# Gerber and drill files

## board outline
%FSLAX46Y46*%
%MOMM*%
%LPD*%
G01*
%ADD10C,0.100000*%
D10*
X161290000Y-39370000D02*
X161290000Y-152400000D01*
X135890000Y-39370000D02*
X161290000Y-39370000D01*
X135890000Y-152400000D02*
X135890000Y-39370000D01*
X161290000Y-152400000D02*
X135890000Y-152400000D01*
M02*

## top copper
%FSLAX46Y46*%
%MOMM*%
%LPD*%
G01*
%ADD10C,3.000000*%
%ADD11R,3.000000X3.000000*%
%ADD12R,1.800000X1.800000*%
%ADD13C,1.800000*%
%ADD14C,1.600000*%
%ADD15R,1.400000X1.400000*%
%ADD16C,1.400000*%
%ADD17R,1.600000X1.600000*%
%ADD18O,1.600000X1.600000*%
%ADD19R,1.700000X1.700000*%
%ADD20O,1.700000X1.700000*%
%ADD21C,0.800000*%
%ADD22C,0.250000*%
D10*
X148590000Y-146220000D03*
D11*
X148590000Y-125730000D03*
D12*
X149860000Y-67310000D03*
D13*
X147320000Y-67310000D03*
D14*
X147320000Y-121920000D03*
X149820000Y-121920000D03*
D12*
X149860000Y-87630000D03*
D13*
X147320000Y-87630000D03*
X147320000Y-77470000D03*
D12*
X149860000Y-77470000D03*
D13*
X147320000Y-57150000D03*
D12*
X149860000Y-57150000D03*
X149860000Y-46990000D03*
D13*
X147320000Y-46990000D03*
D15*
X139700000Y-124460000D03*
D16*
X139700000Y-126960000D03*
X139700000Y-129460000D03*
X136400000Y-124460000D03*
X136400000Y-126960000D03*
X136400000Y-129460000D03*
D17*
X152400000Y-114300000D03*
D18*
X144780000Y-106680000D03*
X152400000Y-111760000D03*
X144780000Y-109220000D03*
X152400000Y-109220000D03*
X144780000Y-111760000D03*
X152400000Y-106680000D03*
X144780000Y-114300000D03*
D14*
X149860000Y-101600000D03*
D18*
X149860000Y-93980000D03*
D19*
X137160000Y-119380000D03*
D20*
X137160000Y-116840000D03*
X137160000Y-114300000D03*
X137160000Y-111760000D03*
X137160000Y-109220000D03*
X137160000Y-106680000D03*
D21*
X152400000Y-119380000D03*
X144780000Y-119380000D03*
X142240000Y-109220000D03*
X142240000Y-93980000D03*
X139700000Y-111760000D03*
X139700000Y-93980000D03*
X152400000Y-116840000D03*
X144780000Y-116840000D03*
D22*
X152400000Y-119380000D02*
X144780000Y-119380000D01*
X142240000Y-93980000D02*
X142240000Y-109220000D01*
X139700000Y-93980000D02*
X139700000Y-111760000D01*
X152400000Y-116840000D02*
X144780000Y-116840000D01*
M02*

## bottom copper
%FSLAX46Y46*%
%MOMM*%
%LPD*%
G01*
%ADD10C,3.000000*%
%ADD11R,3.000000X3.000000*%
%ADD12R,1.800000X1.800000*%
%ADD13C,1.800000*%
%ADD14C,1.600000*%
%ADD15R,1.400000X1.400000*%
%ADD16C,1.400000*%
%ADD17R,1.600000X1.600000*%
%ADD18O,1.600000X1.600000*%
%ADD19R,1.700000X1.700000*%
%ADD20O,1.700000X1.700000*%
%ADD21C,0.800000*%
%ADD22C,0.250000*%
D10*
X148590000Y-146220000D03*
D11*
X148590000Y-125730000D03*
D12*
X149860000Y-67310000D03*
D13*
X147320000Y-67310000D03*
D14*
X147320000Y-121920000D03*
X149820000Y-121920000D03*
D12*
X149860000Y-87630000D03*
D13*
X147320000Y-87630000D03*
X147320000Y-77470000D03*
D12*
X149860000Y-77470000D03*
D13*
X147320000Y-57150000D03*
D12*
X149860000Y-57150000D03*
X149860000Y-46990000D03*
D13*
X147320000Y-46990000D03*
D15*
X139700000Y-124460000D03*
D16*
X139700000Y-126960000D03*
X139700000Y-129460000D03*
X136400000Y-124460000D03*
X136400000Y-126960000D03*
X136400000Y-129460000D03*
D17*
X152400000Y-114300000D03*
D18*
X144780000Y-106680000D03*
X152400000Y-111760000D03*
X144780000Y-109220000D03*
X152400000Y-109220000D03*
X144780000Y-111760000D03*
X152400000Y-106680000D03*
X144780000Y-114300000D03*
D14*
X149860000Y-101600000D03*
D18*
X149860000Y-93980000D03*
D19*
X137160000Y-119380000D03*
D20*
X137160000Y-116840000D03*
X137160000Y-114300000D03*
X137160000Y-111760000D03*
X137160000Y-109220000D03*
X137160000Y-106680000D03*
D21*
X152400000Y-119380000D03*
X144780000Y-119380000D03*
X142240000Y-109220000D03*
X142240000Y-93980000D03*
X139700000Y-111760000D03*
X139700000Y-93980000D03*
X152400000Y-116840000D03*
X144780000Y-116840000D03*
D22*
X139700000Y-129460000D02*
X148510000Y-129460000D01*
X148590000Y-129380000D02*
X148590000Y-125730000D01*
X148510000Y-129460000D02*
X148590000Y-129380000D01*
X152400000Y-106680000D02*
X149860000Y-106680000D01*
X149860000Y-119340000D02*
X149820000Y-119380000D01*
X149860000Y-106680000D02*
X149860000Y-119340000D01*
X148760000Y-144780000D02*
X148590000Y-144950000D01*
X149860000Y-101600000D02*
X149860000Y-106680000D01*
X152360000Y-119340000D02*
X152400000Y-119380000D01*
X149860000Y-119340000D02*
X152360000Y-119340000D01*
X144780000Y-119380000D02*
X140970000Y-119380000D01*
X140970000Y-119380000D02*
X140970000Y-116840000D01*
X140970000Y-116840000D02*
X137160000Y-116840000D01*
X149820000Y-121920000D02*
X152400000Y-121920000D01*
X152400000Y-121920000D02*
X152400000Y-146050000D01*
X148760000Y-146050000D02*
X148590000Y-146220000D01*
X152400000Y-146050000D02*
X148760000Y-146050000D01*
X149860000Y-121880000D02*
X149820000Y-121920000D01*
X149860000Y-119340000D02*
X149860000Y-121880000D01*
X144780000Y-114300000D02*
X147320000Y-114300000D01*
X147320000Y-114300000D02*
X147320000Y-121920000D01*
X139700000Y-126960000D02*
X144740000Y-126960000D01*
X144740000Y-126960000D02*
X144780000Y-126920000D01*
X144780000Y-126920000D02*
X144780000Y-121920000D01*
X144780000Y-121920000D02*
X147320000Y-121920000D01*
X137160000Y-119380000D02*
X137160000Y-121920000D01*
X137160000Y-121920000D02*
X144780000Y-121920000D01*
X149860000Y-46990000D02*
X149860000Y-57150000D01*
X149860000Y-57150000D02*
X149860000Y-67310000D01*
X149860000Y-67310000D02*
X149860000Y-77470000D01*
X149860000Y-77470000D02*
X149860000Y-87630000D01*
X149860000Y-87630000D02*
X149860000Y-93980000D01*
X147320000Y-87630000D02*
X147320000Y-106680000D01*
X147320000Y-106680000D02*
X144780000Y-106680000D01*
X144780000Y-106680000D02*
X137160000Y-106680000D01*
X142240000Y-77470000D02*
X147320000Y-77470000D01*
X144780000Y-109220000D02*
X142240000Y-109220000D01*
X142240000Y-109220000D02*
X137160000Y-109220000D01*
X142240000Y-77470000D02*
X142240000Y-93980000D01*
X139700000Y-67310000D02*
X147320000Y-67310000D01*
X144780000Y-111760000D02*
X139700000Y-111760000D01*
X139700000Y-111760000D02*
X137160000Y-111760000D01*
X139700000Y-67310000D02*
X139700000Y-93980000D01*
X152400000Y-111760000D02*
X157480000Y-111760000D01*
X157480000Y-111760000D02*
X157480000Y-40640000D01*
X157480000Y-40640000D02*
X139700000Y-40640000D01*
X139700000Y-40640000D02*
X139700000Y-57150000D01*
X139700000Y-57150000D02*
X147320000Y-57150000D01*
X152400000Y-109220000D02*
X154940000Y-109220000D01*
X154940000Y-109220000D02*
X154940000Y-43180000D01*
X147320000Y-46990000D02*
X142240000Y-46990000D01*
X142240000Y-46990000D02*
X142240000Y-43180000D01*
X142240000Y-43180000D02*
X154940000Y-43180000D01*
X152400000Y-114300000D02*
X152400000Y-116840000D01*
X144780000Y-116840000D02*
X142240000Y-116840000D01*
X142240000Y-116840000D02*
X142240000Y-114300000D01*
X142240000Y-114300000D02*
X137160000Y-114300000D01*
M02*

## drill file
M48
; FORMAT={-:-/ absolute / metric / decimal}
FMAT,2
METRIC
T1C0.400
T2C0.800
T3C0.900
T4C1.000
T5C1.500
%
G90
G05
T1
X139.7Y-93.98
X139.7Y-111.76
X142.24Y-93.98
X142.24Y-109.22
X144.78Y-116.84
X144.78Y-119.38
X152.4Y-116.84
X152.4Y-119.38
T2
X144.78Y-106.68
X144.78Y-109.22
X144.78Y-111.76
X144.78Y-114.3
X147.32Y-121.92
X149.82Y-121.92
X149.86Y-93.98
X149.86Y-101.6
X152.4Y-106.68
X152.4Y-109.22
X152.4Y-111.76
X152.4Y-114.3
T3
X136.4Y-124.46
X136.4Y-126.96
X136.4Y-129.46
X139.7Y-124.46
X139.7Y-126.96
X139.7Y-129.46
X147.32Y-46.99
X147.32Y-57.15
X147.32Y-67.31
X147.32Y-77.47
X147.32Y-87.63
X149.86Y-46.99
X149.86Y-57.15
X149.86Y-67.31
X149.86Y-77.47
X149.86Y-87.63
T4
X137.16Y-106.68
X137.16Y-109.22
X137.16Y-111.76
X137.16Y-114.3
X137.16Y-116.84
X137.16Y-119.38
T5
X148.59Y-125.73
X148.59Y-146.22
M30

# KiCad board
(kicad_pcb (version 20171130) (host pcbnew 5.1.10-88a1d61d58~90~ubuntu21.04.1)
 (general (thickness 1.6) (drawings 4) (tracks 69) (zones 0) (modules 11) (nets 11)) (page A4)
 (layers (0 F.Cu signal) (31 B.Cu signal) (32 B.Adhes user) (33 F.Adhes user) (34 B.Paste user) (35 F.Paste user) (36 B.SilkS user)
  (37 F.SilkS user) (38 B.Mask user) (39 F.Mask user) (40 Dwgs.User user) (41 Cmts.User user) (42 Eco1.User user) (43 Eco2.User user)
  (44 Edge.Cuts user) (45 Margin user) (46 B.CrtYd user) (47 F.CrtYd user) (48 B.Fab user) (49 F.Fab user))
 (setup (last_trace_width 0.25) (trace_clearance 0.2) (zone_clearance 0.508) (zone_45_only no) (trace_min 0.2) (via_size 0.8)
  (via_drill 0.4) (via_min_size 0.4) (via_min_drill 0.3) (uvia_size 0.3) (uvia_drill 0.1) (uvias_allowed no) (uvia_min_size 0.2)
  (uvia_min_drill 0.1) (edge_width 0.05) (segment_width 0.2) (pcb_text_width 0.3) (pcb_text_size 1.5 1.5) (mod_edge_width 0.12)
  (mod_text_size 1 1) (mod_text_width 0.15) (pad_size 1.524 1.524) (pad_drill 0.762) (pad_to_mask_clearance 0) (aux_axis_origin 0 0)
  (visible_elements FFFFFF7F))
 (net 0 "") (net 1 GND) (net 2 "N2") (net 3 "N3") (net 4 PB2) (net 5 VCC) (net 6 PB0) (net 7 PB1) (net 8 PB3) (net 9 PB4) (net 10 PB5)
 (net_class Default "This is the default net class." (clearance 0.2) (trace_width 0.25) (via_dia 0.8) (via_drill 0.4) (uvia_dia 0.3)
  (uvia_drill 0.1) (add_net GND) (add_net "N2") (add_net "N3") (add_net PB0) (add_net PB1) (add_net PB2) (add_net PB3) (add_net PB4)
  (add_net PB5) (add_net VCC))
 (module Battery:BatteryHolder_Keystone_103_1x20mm (layer F.Cu) (at 148.59 125.73 270)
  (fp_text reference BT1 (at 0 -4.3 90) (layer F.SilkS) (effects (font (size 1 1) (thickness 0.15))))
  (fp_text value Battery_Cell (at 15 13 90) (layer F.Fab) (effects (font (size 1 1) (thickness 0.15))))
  (pad 2 thru_hole circle (at 20.49 0 270) (size 3 3) (drill 1.5) (layers *.Cu *.Mask) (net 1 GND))
  (pad 1 thru_hole rect (at 0 0 270) (size 3 3) (drill 1.5) (layers *.Cu *.Mask) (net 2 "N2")))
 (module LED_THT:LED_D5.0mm (layer F.Cu) (at 149.86 67.31 180)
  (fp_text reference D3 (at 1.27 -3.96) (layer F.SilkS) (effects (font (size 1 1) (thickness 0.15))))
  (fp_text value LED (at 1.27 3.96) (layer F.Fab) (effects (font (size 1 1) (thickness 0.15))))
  (pad 1 thru_hole rect (at 0 0 180) (size 1.8 1.8) (drill 0.9) (layers *.Cu *.Mask) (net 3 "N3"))
  (pad 2 thru_hole circle (at 2.54 0 180) (size 1.8 1.8) (drill 0.9) (layers *.Cu *.Mask) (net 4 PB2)))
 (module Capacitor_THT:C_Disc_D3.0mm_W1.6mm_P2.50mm (layer F.Cu) (at 147.32 121.92)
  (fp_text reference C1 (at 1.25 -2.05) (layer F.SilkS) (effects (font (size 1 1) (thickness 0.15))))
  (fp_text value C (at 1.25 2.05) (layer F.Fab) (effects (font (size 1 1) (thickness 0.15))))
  (pad 1 thru_hole circle (at 0 0) (size 1.6 1.6) (drill 0.8) (layers *.Cu *.Mask) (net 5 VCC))
  (pad 2 thru_hole circle (at 2.5 0) (size 1.6 1.6) (drill 0.8) (layers *.Cu *.Mask) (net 1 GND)))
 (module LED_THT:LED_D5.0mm (layer F.Cu) (at 149.86 87.63 180)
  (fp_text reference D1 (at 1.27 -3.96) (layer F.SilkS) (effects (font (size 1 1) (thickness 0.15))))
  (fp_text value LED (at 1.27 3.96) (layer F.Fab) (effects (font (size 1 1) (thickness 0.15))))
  (pad 1 thru_hole rect (at 0 0 180) (size 1.8 1.8) (drill 0.9) (layers *.Cu *.Mask) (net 3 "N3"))
  (pad 2 thru_hole circle (at 2.54 0 180) (size 1.8 1.8) (drill 0.9) (layers *.Cu *.Mask) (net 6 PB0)))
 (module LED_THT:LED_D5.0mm (layer F.Cu) (at 149.86 77.47 180)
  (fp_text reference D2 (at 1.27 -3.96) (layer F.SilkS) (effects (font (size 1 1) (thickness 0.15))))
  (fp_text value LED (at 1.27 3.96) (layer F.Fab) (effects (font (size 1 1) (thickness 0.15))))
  (pad 2 thru_hole circle (at 2.54 0 180) (size 1.8 1.8) (drill 0.9) (layers *.Cu *.Mask) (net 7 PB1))
  (pad 1 thru_hole rect (at 0 0 180) (size 1.8 1.8) (drill 0.9) (layers *.Cu *.Mask) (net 3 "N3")))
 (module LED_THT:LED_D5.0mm (layer F.Cu) (at 149.86 57.15 180)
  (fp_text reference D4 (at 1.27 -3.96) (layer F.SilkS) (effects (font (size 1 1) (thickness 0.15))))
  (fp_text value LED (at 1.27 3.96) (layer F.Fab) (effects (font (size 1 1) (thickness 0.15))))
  (pad 2 thru_hole circle (at 2.54 0 180) (size 1.8 1.8) (drill 0.9) (layers *.Cu *.Mask) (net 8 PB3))
  (pad 1 thru_hole rect (at 0 0 180) (size 1.8 1.8) (drill 0.9) (layers *.Cu *.Mask) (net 3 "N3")))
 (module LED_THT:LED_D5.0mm (layer F.Cu) (at 149.86 46.99 180)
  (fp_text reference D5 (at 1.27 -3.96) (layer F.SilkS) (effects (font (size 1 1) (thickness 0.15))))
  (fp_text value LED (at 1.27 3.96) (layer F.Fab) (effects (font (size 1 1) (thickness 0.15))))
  (pad 1 thru_hole rect (at 0 0 180) (size 1.8 1.8) (drill 0.9) (layers *.Cu *.Mask) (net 3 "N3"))
  (pad 2 thru_hole circle (at 2.54 0 180) (size 1.8 1.8) (drill 0.9) (layers *.Cu *.Mask) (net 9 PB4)))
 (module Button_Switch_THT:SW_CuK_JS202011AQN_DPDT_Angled (layer F.Cu) (at 139.7 124.46 270)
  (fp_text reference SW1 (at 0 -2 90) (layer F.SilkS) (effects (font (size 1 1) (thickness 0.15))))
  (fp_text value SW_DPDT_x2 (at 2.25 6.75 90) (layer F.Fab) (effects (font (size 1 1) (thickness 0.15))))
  (pad 1 thru_hole rect (at 0 0 270) (size 1.4 1.4) (drill 0.9) (layers *.Cu *.Mask))
  (pad 2 thru_hole circle (at 2.5 0 270) (size 1.4 1.4) (drill 0.9) (layers *.Cu *.Mask) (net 5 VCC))
  (pad 3 thru_hole circle (at 5 0 270) (size 1.4 1.4) (drill 0.9) (layers *.Cu *.Mask) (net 2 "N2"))
  (pad 4 thru_hole circle (at 0 3.3 270) (size 1.4 1.4) (drill 0.9) (layers *.Cu *.Mask))
  (pad 5 thru_hole circle (at 2.5 3.3 270) (size 1.4 1.4) (drill 0.9) (layers *.Cu *.Mask))
  (pad 6 thru_hole circle (at 5 3.3 270) (size 1.4 1.4) (drill 0.9) (layers *.Cu *.Mask)))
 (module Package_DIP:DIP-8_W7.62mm (layer F.Cu) (at 152.4 114.3 180)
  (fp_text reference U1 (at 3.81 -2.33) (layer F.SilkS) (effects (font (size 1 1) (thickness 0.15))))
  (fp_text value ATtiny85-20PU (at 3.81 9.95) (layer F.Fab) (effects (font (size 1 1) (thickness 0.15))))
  (pad 1 thru_hole rect (at 0 0 180) (size 1.6 1.6) (drill 0.8) (layers *.Cu *.Mask) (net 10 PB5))
  (pad 5 thru_hole oval (at 7.62 7.62 180) (size 1.6 1.6) (drill 0.8) (layers *.Cu *.Mask) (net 6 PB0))
  (pad 2 thru_hole oval (at 0 2.54 180) (size 1.6 1.6) (drill 0.8) (layers *.Cu *.Mask) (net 8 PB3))
  (pad 6 thru_hole oval (at 7.62 5.08 180) (size 1.6 1.6) (drill 0.8) (layers *.Cu *.Mask) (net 7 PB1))
  (pad 3 thru_hole oval (at 0 5.08 180) (size 1.6 1.6) (drill 0.8) (layers *.Cu *.Mask) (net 9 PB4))
  (pad 7 thru_hole oval (at 7.62 2.54 180) (size 1.6 1.6) (drill 0.8) (layers *.Cu *.Mask) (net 4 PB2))
  (pad 4 thru_hole oval (at 0 7.62 180) (size 1.6 1.6) (drill 0.8) (layers *.Cu *.Mask) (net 1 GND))
  (pad 8 thru_hole oval (at 7.62 0 180) (size 1.6 1.6) (drill 0.8) (layers *.Cu *.Mask) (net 5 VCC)))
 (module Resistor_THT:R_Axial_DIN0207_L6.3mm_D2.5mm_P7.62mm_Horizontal (layer F.Cu) (at 149.86 101.6 90)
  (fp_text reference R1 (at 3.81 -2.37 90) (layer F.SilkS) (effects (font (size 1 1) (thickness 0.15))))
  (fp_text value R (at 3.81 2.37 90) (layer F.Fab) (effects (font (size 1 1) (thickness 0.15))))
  (pad 1 thru_hole circle (at 0 0 90) (size 1.6 1.6) (drill 0.8) (layers *.Cu *.Mask) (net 1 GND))
  (pad 2 thru_hole oval (at 7.62 0 90) (size 1.6 1.6) (drill 0.8) (layers *.Cu *.Mask) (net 3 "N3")))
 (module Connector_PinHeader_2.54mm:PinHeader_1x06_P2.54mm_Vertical (layer F.Cu) (at 137.16 119.38 180)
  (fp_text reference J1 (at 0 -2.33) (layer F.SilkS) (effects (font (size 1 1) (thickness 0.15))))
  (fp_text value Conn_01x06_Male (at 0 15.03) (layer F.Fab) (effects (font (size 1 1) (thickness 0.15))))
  (pad 1 thru_hole rect (at 0 0 180) (size 1.7 1.7) (drill 1) (layers *.Cu *.Mask) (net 5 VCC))
  (pad 2 thru_hole oval (at 0 2.54 180) (size 1.7 1.7) (drill 1) (layers *.Cu *.Mask) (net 1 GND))
  (pad 3 thru_hole oval (at 0 5.08 180) (size 1.7 1.7) (drill 1) (layers *.Cu *.Mask) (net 10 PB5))
  (pad 4 thru_hole oval (at 0 7.62 180) (size 1.7 1.7) (drill 1) (layers *.Cu *.Mask) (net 4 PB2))
  (pad 5 thru_hole oval (at 0 10.16 180) (size 1.7 1.7) (drill 1) (layers *.Cu *.Mask) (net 7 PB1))
  (pad 6 thru_hole oval (at 0 12.7 180) (size 1.7 1.7) (drill 1) (layers *.Cu *.Mask) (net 6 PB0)))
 (gr_line (start 161.29 39.37) (end 161.29 152.4) (layer Edge.Cuts) (width 0.1))
 (gr_line (start 135.89 39.37) (end 161.29 39.37) (layer Edge.Cuts) (width 0.1))
 (gr_line (start 135.89 152.4) (end 135.89 39.37) (layer Edge.Cuts) (width 0.1))
 (gr_line (start 161.29 152.4) (end 135.89 152.4) (layer Edge.Cuts) (width 0.1))
 (segment (start 139.7 129.46) (end 148.51 129.46) (width 0.25) (layer B.Cu) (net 2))
 (segment (start 148.59 129.38) (end 148.59 125.73) (width 0.25) (layer B.Cu) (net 2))
 (segment (start 148.51 129.46) (end 148.59 129.38) (width 0.25) (layer B.Cu) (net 2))
 (segment (start 152.4 106.68) (end 149.86 106.68) (width 0.25) (layer B.Cu) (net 1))
 (segment (start 149.86 119.34) (end 149.82 119.38) (width 0.25) (layer B.Cu) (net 1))
 (segment (start 149.86 106.68) (end 149.86 119.34) (width 0.25) (layer B.Cu) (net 1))
 (segment (start 148.76 144.78) (end 148.59 144.95) (width 0.25) (layer B.Cu) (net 1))
 (segment (start 149.86 101.6) (end 149.86 106.68) (width 0.25) (layer B.Cu) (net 1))
 (via (at 152.4 119.38) (size 0.8) (drill 0.4) (layers F.Cu B.Cu) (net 1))
 (segment (start 152.36 119.34) (end 152.4 119.38) (width 0.25) (layer B.Cu) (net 1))
 (segment (start 149.86 119.34) (end 152.36 119.34) (width 0.25) (layer B.Cu) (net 1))
 (via (at 144.78 119.38) (size 0.8) (drill 0.4) (layers F.Cu B.Cu) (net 1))
 (segment (start 152.4 119.38) (end 144.78 119.38) (width 0.25) (layer F.Cu) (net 1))
 (segment (start 144.78 119.38) (end 140.97 119.38) (width 0.25) (layer B.Cu) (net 1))
 (segment (start 140.97 119.38) (end 140.97 116.84) (width 0.25) (layer B.Cu) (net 1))
 (segment (start 140.97 116.84) (end 137.16 116.84) (width 0.25) (layer B.Cu) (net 1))
 (segment (start 149.82 121.92) (end 152.4 121.92) (width 0.25) (layer B.Cu) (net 1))
 (segment (start 152.4 121.92) (end 152.4 146.05) (width 0.25) (layer B.Cu) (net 1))
 (segment (start 148.76 146.05) (end 148.59 146.22) (width 0.25) (layer B.Cu) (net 1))
 (segment (start 152.4 146.05) (end 148.76 146.05) (width 0.25) (layer B.Cu) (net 1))
 (segment (start 149.86 121.88) (end 149.82 121.92) (width 0.25) (layer B.Cu) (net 1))
 (segment (start 149.86 119.34) (end 149.86 121.88) (width 0.25) (layer B.Cu) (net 1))
 (segment (start 144.78 114.3) (end 147.32 114.3) (width 0.25) (layer B.Cu) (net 5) (status 10))
 (segment (start 147.32 114.3) (end 147.32 121.92) (width 0.25) (layer B.Cu) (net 5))
 (segment (start 139.7 126.96) (end 144.74 126.96) (width 0.25) (layer B.Cu) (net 5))
 (segment (start 144.74 126.96) (end 144.78 126.92) (width 0.25) (layer B.Cu) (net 5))
 (segment (start 144.78 126.92) (end 144.78 121.92) (width 0.25) (layer B.Cu) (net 5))
 (segment (start 144.78 121.92) (end 147.32 121.92) (width 0.25) (layer B.Cu) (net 5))
 (segment (start 137.16 119.38) (end 137.16 121.92) (width 0.25) (layer B.Cu) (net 5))
 (segment (start 137.16 121.92) (end 144.78 121.92) (width 0.25) (layer B.Cu) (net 5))
 (segment (start 149.86 46.99) (end 149.86 57.15) (width 0.25) (layer B.Cu) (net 3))
 (segment (start 149.86 57.15) (end 149.86 67.31) (width 0.25) (layer B.Cu) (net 3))
 (segment (start 149.86 67.31) (end 149.86 77.47) (width 0.25) (layer B.Cu) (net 3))
 (segment (start 149.86 77.47) (end 149.86 87.63) (width 0.25) (layer B.Cu) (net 3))
 (segment (start 149.86 87.63) (end 149.86 93.98) (width 0.25) (layer B.Cu) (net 3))
 (segment (start 147.32 87.63) (end 147.32 106.68) (width 0.25) (layer B.Cu) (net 6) (status 10))
 (segment (start 147.32 106.68) (end 144.78 106.68) (width 0.25) (layer B.Cu) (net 6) (status 20))
 (segment (start 144.78 106.68) (end 137.16 106.68) (width 0.25) (layer B.Cu) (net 6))
 (segment (start 142.24 77.47) (end 147.32 77.47) (width 0.25) (layer B.Cu) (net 7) (status 20))
 (segment (start 144.78 109.22) (end 142.24 109.22) (width 0.25) (layer B.Cu) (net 7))
 (segment (start 142.24 109.22) (end 137.16 109.22) (width 0.25) (layer B.Cu) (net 7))
 (via (at 142.24 109.22) (size 0.8) (drill 0.4) (layers F.Cu B.Cu) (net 7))
 (via (at 142.24 93.98) (size 0.8) (drill 0.4) (layers F.Cu B.Cu) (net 7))
 (segment (start 142.24 77.47) (end 142.24 93.98) (width 0.25) (layer B.Cu) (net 7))
 (segment (start 142.24 93.98) (end 142.24 109.22) (width 0.25) (layer F.Cu) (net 7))
 (segment (start 139.7 67.31) (end 147.32 67.31) (width 0.25) (layer B.Cu) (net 4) (status 20))
 (segment (start 144.78 111.76) (end 139.7 111.76) (width 0.25) (layer B.Cu) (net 4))
 (segment (start 139.7 111.76) (end 137.16 111.76) (width 0.25) (layer B.Cu) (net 4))
 (via (at 139.7 111.76) (size 0.8) (drill 0.4) (layers F.Cu B.Cu) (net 4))
 (via (at 139.7 93.98) (size 0.8) (drill 0.4) (layers F.Cu B.Cu) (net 4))
 (segment (start 139.7 67.31) (end 139.7 93.98) (width 0.25) (layer B.Cu) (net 4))
 (segment (start 139.7 93.98) (end 139.7 111.76) (width 0.25) (layer F.Cu) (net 4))
 (segment (start 152.4 111.76) (end 157.48 111.76) (width 0.25) (layer B.Cu) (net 8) (status 10))
 (segment (start 157.48 111.76) (end 157.48 40.64) (width 0.25) (layer B.Cu) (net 8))
 (segment (start 157.48 40.64) (end 139.7 40.64) (width 0.25) (layer B.Cu) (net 8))
 (segment (start 139.7 40.64) (end 139.7 57.15) (width 0.25) (layer B.Cu) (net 8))
 (segment (start 139.7 57.15) (end 147.32 57.15) (width 0.25) (layer B.Cu) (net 8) (status 20))
 (segment (start 152.4 109.22) (end 154.94 109.22) (width 0.25) (layer B.Cu) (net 9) (status 10))
 (segment (start 154.94 109.22) (end 154.94 43.18) (width 0.25) (layer B.Cu) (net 9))
 (segment (start 147.32 46.99) (end 142.24 46.99) (width 0.25) (layer B.Cu) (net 9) (status 10))
 (segment (start 142.24 46.99) (end 142.24 43.18) (width 0.25) (layer B.Cu) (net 9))
 (segment (start 142.24 43.18) (end 154.94 43.18) (width 0.25) (layer B.Cu) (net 9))
 (via (at 152.4 116.84) (size 0.8) (drill 0.4) (layers F.Cu B.Cu) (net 10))
 (segment (start 152.4 114.3) (end 152.4 116.84) (width 0.25) (layer B.Cu) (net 10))
 (via (at 144.78 116.84) (size 0.8) (drill 0.4) (layers F.Cu B.Cu) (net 10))
 (segment (start 152.4 116.84) (end 144.78 116.84) (width 0.25) (layer F.Cu) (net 10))
 (segment (start 144.78 116.84) (end 142.24 116.84) (width 0.25) (layer B.Cu) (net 10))
 (segment (start 142.24 116.84) (end 142.24 114.3) (width 0.25) (layer B.Cu) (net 10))
 (segment (start 142.24 114.3) (end 137.16 114.3) (width 0.25) (layer B.Cu) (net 10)))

